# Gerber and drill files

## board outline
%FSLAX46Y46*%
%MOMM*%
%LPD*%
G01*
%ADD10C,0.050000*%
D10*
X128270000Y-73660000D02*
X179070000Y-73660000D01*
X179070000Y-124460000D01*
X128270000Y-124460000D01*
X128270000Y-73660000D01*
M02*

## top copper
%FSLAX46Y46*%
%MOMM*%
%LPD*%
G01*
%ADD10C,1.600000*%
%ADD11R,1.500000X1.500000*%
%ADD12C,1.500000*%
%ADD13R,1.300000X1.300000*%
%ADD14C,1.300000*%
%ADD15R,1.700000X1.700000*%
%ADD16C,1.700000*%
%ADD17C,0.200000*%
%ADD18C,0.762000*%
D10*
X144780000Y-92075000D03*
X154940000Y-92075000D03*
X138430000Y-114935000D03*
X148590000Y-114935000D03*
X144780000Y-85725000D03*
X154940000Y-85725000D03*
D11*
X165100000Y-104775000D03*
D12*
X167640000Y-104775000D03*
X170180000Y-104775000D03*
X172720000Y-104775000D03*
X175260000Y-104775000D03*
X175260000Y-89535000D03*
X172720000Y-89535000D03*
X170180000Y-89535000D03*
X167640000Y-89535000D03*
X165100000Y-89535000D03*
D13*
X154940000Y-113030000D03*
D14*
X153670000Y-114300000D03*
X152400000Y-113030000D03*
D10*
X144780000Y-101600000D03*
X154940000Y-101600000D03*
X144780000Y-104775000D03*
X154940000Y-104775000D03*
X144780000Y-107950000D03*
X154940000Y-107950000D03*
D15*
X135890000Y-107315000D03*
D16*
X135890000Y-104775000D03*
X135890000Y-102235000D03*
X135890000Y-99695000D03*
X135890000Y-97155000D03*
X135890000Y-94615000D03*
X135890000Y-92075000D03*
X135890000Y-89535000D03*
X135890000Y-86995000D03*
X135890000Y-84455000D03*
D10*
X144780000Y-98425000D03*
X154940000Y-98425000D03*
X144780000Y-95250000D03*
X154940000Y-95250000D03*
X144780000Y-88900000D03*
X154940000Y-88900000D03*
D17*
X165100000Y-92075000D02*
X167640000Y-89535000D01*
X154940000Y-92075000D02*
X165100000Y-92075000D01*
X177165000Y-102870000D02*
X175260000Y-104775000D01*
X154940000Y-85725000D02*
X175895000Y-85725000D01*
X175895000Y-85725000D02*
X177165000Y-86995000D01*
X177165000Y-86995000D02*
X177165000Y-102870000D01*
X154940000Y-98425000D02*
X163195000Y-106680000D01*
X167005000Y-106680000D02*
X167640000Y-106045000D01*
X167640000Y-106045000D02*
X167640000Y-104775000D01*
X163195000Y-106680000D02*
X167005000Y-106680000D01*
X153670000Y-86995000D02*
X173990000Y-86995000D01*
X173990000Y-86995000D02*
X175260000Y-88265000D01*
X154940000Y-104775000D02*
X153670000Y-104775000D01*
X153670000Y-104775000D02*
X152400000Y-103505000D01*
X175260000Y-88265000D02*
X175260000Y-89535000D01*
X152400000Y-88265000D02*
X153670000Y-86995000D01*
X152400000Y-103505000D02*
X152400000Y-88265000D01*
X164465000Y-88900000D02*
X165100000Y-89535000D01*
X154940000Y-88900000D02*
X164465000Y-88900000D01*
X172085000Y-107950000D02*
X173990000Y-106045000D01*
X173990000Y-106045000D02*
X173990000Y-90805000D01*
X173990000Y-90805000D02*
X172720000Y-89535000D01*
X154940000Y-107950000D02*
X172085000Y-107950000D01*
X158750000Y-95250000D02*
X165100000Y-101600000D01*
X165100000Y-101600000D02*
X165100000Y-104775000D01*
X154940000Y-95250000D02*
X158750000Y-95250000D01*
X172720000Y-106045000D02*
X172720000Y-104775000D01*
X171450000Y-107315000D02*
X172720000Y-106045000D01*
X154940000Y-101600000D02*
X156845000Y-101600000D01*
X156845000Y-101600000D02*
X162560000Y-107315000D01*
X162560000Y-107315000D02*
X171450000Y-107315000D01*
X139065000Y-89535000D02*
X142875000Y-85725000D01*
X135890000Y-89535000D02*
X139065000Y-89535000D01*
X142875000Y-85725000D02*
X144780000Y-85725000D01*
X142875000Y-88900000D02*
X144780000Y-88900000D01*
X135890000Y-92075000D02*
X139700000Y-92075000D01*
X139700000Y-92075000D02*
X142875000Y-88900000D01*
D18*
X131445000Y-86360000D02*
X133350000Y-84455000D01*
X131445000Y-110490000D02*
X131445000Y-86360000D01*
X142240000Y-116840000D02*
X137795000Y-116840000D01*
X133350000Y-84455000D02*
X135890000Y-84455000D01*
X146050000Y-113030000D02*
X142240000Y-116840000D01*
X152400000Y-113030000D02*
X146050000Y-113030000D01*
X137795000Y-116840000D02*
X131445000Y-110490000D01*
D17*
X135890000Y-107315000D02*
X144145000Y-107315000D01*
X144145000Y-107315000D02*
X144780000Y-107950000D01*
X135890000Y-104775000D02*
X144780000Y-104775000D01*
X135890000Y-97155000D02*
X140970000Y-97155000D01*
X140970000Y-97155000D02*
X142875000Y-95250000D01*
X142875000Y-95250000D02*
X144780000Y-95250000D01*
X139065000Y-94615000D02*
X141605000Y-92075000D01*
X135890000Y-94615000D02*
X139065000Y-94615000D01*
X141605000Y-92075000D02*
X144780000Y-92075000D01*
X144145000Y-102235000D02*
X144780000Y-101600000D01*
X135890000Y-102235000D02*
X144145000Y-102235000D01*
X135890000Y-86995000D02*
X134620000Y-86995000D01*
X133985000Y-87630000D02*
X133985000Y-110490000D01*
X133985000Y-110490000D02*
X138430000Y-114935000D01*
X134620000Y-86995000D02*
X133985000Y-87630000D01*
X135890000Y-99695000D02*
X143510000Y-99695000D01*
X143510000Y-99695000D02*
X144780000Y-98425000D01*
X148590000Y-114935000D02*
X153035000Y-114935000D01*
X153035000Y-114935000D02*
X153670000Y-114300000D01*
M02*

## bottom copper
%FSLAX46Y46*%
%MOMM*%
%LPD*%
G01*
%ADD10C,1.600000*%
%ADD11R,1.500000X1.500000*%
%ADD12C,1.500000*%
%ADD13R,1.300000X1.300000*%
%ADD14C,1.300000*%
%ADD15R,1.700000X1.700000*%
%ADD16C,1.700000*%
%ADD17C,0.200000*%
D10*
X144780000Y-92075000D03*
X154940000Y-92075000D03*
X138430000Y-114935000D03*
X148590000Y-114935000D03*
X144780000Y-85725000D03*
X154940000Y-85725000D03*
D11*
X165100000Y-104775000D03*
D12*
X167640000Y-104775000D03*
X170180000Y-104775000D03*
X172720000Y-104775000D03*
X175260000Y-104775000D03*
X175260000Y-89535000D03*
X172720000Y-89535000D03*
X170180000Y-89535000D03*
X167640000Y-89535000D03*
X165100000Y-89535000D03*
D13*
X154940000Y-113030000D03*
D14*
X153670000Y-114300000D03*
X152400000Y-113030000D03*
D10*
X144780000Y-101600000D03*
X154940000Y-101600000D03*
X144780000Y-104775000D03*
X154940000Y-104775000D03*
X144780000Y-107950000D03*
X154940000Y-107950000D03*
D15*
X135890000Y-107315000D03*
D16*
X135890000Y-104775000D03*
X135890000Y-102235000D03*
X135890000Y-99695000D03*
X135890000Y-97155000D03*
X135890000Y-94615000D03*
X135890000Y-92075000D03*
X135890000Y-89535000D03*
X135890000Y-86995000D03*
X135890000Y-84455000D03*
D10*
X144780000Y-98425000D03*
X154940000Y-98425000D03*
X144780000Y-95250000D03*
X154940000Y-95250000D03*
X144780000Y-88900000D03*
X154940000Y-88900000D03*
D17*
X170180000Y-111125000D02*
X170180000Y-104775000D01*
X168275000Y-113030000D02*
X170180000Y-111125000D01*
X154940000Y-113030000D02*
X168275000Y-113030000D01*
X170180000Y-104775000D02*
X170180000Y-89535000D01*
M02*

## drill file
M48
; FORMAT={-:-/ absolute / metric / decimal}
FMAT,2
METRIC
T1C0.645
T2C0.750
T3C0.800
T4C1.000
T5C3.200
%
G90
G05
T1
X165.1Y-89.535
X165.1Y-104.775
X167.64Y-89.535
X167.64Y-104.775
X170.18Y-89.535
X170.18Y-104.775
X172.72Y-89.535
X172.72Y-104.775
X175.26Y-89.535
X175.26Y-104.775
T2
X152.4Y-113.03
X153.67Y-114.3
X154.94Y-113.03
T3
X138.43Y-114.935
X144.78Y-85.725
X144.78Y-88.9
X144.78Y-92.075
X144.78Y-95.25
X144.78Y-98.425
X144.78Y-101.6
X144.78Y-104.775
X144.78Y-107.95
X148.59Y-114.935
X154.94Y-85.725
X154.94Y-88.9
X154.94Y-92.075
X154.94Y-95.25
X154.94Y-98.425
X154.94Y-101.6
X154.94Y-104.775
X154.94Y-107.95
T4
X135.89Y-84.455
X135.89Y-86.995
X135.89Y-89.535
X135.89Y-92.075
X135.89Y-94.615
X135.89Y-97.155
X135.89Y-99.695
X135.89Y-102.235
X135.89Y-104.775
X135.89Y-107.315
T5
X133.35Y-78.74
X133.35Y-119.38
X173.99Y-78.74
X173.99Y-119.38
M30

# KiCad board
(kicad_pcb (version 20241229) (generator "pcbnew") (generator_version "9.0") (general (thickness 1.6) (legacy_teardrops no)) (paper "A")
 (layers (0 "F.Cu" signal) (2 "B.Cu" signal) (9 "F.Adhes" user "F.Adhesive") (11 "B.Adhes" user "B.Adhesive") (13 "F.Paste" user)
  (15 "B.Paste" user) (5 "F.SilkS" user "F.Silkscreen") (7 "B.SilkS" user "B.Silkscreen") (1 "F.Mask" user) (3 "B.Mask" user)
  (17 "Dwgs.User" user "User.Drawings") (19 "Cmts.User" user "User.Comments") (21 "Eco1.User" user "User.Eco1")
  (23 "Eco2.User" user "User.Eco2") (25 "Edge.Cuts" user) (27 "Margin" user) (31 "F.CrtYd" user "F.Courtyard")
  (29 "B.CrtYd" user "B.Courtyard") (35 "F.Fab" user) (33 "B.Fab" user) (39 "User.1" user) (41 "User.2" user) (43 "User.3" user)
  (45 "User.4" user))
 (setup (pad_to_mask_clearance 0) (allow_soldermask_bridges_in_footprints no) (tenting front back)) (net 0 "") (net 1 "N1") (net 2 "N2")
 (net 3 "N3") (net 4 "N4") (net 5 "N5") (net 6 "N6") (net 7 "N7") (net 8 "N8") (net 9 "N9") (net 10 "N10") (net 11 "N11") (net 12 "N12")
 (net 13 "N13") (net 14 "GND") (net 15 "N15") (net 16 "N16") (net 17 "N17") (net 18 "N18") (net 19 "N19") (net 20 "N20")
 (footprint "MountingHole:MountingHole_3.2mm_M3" (layer "F.Cu") (at 133.35 78.74)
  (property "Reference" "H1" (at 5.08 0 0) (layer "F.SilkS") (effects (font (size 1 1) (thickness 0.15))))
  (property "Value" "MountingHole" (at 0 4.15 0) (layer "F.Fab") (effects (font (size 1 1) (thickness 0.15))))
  (pad "" np_thru_hole circle (at 0 0) (size 3.2 3.2) (drill 3.2) (layers "*.Cu" "*.Mask")))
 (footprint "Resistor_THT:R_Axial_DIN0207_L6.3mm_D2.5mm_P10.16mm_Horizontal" (layer "F.Cu") (at 144.78 92.075)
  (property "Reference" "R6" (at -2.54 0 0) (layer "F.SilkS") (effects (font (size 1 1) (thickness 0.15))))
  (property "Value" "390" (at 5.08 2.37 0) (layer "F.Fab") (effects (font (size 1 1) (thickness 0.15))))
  (pad "1" thru_hole circle (at 0 0) (size 1.6 1.6) (drill 0.8) (layers "*.Cu" "*.Mask") (remove_unused_layers no) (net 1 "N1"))
  (pad "2" thru_hole circle (at 10.16 0) (size 1.6 1.6) (drill 0.8) (layers "*.Cu" "*.Mask") (remove_unused_layers no) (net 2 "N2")))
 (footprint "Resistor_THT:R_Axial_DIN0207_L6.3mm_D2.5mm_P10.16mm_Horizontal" (layer "F.Cu") (at 138.43 114.935)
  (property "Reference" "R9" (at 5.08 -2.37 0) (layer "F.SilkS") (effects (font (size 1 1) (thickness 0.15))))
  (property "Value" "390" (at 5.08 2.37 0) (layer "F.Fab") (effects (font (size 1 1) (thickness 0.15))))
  (pad "1" thru_hole circle (at 0 0) (size 1.6 1.6) (drill 0.8) (layers "*.Cu" "*.Mask") (remove_unused_layers no) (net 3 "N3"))
  (pad "2" thru_hole circle (at 10.16 0) (size 1.6 1.6) (drill 0.8) (layers "*.Cu" "*.Mask") (remove_unused_layers no) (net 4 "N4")))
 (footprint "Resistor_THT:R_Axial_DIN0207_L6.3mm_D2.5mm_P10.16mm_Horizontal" (layer "F.Cu") (at 144.78 85.725)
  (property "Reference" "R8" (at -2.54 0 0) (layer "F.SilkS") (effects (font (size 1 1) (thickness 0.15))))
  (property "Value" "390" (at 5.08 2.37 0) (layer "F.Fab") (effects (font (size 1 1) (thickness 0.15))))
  (pad "1" thru_hole circle (at 0 0) (size 1.6 1.6) (drill 0.8) (layers "*.Cu" "*.Mask") (remove_unused_layers no) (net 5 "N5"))
  (pad "2" thru_hole circle (at 10.16 0) (size 1.6 1.6) (drill 0.8) (layers "*.Cu" "*.Mask") (remove_unused_layers no) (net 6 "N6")))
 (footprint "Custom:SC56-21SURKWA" (layer "F.Cu") (at 170.18 97.155)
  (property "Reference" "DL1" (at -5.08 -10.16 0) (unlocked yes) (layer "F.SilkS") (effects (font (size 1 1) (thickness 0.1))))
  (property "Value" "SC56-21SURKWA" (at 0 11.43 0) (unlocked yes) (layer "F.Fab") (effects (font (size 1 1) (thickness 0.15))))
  (pad "1" thru_hole rect (at -5.08 7.62 90) (size 1.5 1.5) (drill 0.64516) (layers "*.Cu" "*.Mask") (remove_unused_layers no) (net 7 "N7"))
  (pad "2" thru_hole circle (at -2.54 7.62 90) (size 1.5 1.5) (drill 0.64516) (layers "*.Cu" "*.Mask") (remove_unused_layers no)
   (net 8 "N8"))
  (pad "3" thru_hole circle (at 0 7.62 90) (size 1.5 1.5) (drill 0.64516) (layers "*.Cu" "*.Mask") (remove_unused_layers no) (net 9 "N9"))
  (pad "4" thru_hole circle (at 2.54 7.62 90) (size 1.5 1.5) (drill 0.64516) (layers "*.Cu" "*.Mask") (remove_unused_layers no)
   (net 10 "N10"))
  (pad "5" thru_hole circle (at 5.08 7.62 90) (size 1.5 1.5) (drill 0.64516) (layers "*.Cu" "*.Mask") (remove_unused_layers no) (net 6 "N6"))
  (pad "6" thru_hole circle (at 5.08 -7.62 90) (size 1.5 1.5) (drill 0.64516) (layers "*.Cu" "*.Mask") (remove_unused_layers no)
   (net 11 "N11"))
  (pad "7" thru_hole circle (at 2.54 -7.62 90) (size 1.5 1.5) (drill 0.64516) (layers "*.Cu" "*.Mask") (remove_unused_layers no)
   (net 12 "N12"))
  (pad "8" thru_hole circle (at 0 -7.62 90) (size 1.5 1.5) (drill 0.64516) (layers "*.Cu" "*.Mask") (remove_unused_layers no) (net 9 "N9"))
  (pad "9" thru_hole circle (at -2.54 -7.62 90) (size 1.5 1.5) (drill 0.64516) (layers "*.Cu" "*.Mask") (remove_unused_layers no)
   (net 2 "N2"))
  (pad "10" thru_hole circle (at -5.08 -7.62 90) (size 1.5 1.5) (drill 0.64516) (layers "*.Cu" "*.Mask") (remove_unused_layers no)
   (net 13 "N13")))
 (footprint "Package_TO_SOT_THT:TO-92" (layer "F.Cu") (at 154.94 113.03 180)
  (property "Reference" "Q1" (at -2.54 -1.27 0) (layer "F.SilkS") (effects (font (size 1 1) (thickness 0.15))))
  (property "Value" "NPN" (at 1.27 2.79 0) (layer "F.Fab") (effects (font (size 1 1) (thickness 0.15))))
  (pad "1" thru_hole rect (at 0 0 180) (size 1.3 1.3) (drill 0.75) (layers "*.Cu" "*.Mask") (remove_unused_layers no) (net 9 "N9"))
  (pad "2" thru_hole circle (at 1.27 -1.27 180) (size 1.3 1.3) (drill 0.75) (layers "*.Cu" "*.Mask") (remove_unused_layers no) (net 4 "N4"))
  (pad "3" thru_hole circle (at 2.54 0 180) (size 1.3 1.3) (drill 0.75) (layers "*.Cu" "*.Mask") (remove_unused_layers no) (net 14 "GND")))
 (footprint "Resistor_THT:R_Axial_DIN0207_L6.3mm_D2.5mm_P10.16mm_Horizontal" (layer "F.Cu") (at 144.78 101.6)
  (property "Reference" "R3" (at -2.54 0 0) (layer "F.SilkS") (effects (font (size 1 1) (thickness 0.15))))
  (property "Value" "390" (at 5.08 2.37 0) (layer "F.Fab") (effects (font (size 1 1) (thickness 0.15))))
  (pad "1" thru_hole circle (at 0 0) (size 1.6 1.6) (drill 0.8) (layers "*.Cu" "*.Mask") (remove_unused_layers no) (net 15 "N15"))
  (pad "2" thru_hole circle (at 10.16 0) (size 1.6 1.6) (drill 0.8) (layers "*.Cu" "*.Mask") (remove_unused_layers no) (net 10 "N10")))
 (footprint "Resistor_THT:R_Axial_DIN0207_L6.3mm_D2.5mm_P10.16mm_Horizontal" (layer "F.Cu") (at 144.78 104.775)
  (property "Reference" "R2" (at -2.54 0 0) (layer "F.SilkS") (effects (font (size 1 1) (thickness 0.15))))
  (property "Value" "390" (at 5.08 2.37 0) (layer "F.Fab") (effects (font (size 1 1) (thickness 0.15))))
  (pad "1" thru_hole circle (at 0 0) (size 1.6 1.6) (drill 0.8) (layers "*.Cu" "*.Mask") (remove_unused_layers no) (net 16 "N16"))
  (pad "2" thru_hole circle (at 10.16 0) (size 1.6 1.6) (drill 0.8) (layers "*.Cu" "*.Mask") (remove_unused_layers no) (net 11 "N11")))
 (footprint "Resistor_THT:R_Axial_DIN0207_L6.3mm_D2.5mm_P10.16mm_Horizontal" (layer "F.Cu") (at 144.78 107.95)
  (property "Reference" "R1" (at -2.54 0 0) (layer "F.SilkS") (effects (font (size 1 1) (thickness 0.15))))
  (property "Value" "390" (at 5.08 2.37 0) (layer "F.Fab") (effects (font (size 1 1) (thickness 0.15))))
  (pad "1" thru_hole circle (at 0 0) (size 1.6 1.6) (drill 0.8) (layers "*.Cu" "*.Mask") (remove_unused_layers no) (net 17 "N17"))
  (pad "2" thru_hole circle (at 10.16 0) (size 1.6 1.6) (drill 0.8) (layers "*.Cu" "*.Mask") (remove_unused_layers no) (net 12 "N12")))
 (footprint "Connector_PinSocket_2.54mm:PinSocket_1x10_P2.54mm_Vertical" (layer "F.Cu") (at 135.89 107.315 180)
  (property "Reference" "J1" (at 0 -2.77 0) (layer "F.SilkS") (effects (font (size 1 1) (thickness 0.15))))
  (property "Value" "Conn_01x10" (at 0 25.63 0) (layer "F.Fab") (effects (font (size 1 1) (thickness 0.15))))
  (pad "1" thru_hole rect (at 0 0 180) (size 1.7 1.7) (drill 1) (layers "*.Cu" "*.Mask") (remove_unused_layers no) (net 17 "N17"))
  (pad "2" thru_hole circle (at 0 2.54 180) (size 1.7 1.7) (drill 1) (layers "*.Cu" "*.Mask") (remove_unused_layers no) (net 16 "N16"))
  (pad "3" thru_hole circle (at 0 5.08 180) (size 1.7 1.7) (drill 1) (layers "*.Cu" "*.Mask") (remove_unused_layers no) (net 15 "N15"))
  (pad "4" thru_hole circle (at 0 7.62 180) (size 1.7 1.7) (drill 1) (layers "*.Cu" "*.Mask") (remove_unused_layers no) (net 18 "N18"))
  (pad "5" thru_hole circle (at 0 10.16 180) (size 1.7 1.7) (drill 1) (layers "*.Cu" "*.Mask") (remove_unused_layers no) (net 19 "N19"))
  (pad "6" thru_hole circle (at 0 12.7 180) (size 1.7 1.7) (drill 1) (layers "*.Cu" "*.Mask") (remove_unused_layers no) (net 1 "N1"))
  (pad "7" thru_hole circle (at 0 15.24 180) (size 1.7 1.7) (drill 1) (layers "*.Cu" "*.Mask") (remove_unused_layers no) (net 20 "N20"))
  (pad "8" thru_hole circle (at 0 17.78 180) (size 1.7 1.7) (drill 1) (layers "*.Cu" "*.Mask") (remove_unused_layers no) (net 5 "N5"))
  (pad "9" thru_hole circle (at 0 20.32 180) (size 1.7 1.7) (drill 1) (layers "*.Cu" "*.Mask") (remove_unused_layers no) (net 3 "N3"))
  (pad "10" thru_hole circle (at 0 22.86 180) (size 1.7 1.7) (drill 1) (layers "*.Cu" "*.Mask") (remove_unused_layers no) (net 14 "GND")))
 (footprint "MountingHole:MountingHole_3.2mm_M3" (layer "F.Cu") (at 173.99 78.74)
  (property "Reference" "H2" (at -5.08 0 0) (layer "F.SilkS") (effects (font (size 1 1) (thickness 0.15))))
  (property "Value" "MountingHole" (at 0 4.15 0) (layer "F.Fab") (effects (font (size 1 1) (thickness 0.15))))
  (pad "" np_thru_hole circle (at 0 0) (size 3.2 3.2) (drill 3.2) (layers "*.Cu" "*.Mask")))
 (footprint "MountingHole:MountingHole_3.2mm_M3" (layer "F.Cu") (at 173.99 119.38)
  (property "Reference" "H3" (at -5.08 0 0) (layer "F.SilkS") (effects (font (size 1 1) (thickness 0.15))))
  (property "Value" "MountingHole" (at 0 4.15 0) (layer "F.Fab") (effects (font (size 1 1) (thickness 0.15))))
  (pad "" np_thru_hole circle (at 0 0) (size 3.2 3.2) (drill 3.2) (layers "*.Cu" "*.Mask")))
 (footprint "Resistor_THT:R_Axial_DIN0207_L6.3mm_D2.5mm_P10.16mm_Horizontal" (layer "F.Cu") (at 144.78 98.425)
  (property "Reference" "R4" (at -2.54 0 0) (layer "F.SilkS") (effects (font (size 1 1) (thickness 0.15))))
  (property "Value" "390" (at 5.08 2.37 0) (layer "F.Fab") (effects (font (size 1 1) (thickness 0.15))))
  (pad "1" thru_hole circle (at 0 0) (size 1.6 1.6) (drill 0.8) (layers "*.Cu" "*.Mask") (remove_unused_layers no) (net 18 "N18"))
  (pad "2" thru_hole circle (at 10.16 0) (size 1.6 1.6) (drill 0.8) (layers "*.Cu" "*.Mask") (remove_unused_layers no) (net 8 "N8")))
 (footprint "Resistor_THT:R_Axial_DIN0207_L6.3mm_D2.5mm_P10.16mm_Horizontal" (layer "F.Cu") (at 144.78 95.25)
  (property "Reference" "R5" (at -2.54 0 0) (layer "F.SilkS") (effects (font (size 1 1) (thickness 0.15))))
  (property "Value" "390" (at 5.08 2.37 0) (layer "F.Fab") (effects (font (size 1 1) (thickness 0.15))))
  (pad "1" thru_hole circle (at 0 0) (size 1.6 1.6) (drill 0.8) (layers "*.Cu" "*.Mask") (remove_unused_layers no) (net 19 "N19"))
  (pad "2" thru_hole circle (at 10.16 0) (size 1.6 1.6) (drill 0.8) (layers "*.Cu" "*.Mask") (remove_unused_layers no) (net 7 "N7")))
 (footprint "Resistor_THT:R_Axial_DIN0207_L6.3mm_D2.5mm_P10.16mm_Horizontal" (layer "F.Cu") (at 144.78 88.9)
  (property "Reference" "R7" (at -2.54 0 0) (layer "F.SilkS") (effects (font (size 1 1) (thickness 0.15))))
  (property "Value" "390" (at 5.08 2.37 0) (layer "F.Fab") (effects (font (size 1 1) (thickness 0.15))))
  (pad "1" thru_hole circle (at 0 0) (size 1.6 1.6) (drill 0.8) (layers "*.Cu" "*.Mask") (remove_unused_layers no) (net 20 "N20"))
  (pad "2" thru_hole circle (at 10.16 0) (size 1.6 1.6) (drill 0.8) (layers "*.Cu" "*.Mask") (remove_unused_layers no) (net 13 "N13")))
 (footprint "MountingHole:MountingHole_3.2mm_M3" (layer "F.Cu") (at 133.35 119.38)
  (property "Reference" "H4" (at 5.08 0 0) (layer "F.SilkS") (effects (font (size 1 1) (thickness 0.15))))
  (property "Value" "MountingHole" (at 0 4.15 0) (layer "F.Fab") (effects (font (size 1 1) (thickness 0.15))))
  (pad "" np_thru_hole circle (at 0 0) (size 3.2 3.2) (drill 3.2) (layers "*.Cu" "*.Mask")))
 (gr_rect (start 128.27 73.66) (end 179.07 124.46) (stroke (width 0.05) (type default)) (fill no) (layer "Edge.Cuts"))
 (segment (start 165.1 92.075) (end 167.64 89.535) (width 0.2) (layer "F.Cu") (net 2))
 (segment (start 154.94 92.075) (end 165.1 92.075) (width 0.2) (layer "F.Cu") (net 2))
 (segment (start 177.165 102.87) (end 175.26 104.775) (width 0.2) (layer "F.Cu") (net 6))
 (segment (start 154.94 85.725) (end 175.895 85.725) (width 0.2) (layer "F.Cu") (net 6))
 (segment (start 175.895 85.725) (end 177.165 86.995) (width 0.2) (layer "F.Cu") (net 6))
 (segment (start 177.165 86.995) (end 177.165 102.87) (width 0.2) (layer "F.Cu") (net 6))
 (segment (start 170.18 111.125) (end 170.18 104.775) (width 0.2) (layer "B.Cu") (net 9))
 (segment (start 168.275 113.03) (end 170.18 111.125) (width 0.2) (layer "B.Cu") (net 9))
 (segment (start 154.94 113.03) (end 168.275 113.03) (width 0.2) (layer "B.Cu") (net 9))
 (segment (start 170.18 104.775) (end 170.18 89.535) (width 0.2) (layer "B.Cu") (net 9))
 (segment (start 154.94 98.425) (end 163.195 106.68) (width 0.2) (layer "F.Cu") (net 8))
 (segment (start 167.005 106.68) (end 167.64 106.045) (width 0.2) (layer "F.Cu") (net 8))
 (segment (start 167.64 106.045) (end 167.64 104.775) (width 0.2) (layer "F.Cu") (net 8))
 (segment (start 163.195 106.68) (end 167.005 106.68) (width 0.2) (layer "F.Cu") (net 8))
 (segment (start 153.67 86.995) (end 173.99 86.995) (width 0.2) (layer "F.Cu") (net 11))
 (segment (start 173.99 86.995) (end 175.26 88.265) (width 0.2) (layer "F.Cu") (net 11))
 (segment (start 154.94 104.775) (end 153.67 104.775) (width 0.2) (layer "F.Cu") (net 11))
 (segment (start 153.67 104.775) (end 152.4 103.505) (width 0.2) (layer "F.Cu") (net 11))
 (segment (start 175.26 88.265) (end 175.26 89.535) (width 0.2) (layer "F.Cu") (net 11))
 (segment (start 152.4 88.265) (end 153.67 86.995) (width 0.2) (layer "F.Cu") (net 11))
 (segment (start 152.4 103.505) (end 152.4 88.265) (width 0.2) (layer "F.Cu") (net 11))
 (segment (start 164.465 88.9) (end 165.1 89.535) (width 0.2) (layer "F.Cu") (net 13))
 (segment (start 154.94 88.9) (end 164.465 88.9) (width 0.2) (layer "F.Cu") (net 13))
 (segment (start 172.085 107.95) (end 173.99 106.045) (width 0.2) (layer "F.Cu") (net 12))
 (segment (start 173.99 106.045) (end 173.99 90.805) (width 0.2) (layer "F.Cu") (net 12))
 (segment (start 173.99 90.805) (end 172.72 89.535) (width 0.2) (layer "F.Cu") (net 12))
 (segment (start 154.94 107.95) (end 172.085 107.95) (width 0.2) (layer "F.Cu") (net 12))
 (segment (start 158.75 95.25) (end 165.1 101.6) (width 0.2) (layer "F.Cu") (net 7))
 (segment (start 165.1 101.6) (end 165.1 104.775) (width 0.2) (layer "F.Cu") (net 7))
 (segment (start 154.94 95.25) (end 158.75 95.25) (width 0.2) (layer "F.Cu") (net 7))
 (segment (start 172.72 106.045) (end 172.72 104.775) (width 0.2) (layer "F.Cu") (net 10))
 (segment (start 171.45 107.315) (end 172.72 106.045) (width 0.2) (layer "F.Cu") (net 10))
 (segment (start 154.94 101.6) (end 156.845 101.6) (width 0.2) (layer "F.Cu") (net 10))
 (segment (start 156.845 101.6) (end 162.56 107.315) (width 0.2) (layer "F.Cu") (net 10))
 (segment (start 162.56 107.315) (end 171.45 107.315) (width 0.2) (layer "F.Cu") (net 10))
 (segment (start 139.065 89.535) (end 142.875 85.725) (width 0.2) (layer "F.Cu") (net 5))
 (segment (start 135.89 89.535) (end 139.065 89.535) (width 0.2) (layer "F.Cu") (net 5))
 (segment (start 142.875 85.725) (end 144.78 85.725) (width 0.2) (layer "F.Cu") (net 5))
 (segment (start 142.875 88.9) (end 144.78 88.9) (width 0.2) (layer "F.Cu") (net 20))
 (segment (start 135.89 92.075) (end 139.7 92.075) (width 0.2) (layer "F.Cu") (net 20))
 (segment (start 139.7 92.075) (end 142.875 88.9) (width 0.2) (layer "F.Cu") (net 20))
 (segment (start 131.445 86.36) (end 133.35 84.455) (width 0.762) (layer "F.Cu") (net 14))
 (segment (start 131.445 110.49) (end 131.445 86.36) (width 0.762) (layer "F.Cu") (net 14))
 (segment (start 142.24 116.84) (end 137.795 116.84) (width 0.762) (layer "F.Cu") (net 14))
 (segment (start 133.35 84.455) (end 135.89 84.455) (width 0.762) (layer "F.Cu") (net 14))
 (segment (start 146.05 113.03) (end 142.24 116.84) (width 0.762) (layer "F.Cu") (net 14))
 (segment (start 152.4 113.03) (end 146.05 113.03) (width 0.762) (layer "F.Cu") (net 14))
 (segment (start 137.795 116.84) (end 131.445 110.49) (width 0.762) (layer "F.Cu") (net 14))
 (segment (start 135.89 107.315) (end 144.145 107.315) (width 0.2) (layer "F.Cu") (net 17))
 (segment (start 144.145 107.315) (end 144.78 107.95) (width 0.2) (layer "F.Cu") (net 17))
 (segment (start 135.89 104.775) (end 144.78 104.775) (width 0.2) (layer "F.Cu") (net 16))
 (segment (start 135.89 97.155) (end 140.97 97.155) (width 0.2) (layer "F.Cu") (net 19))
 (segment (start 140.97 97.155) (end 142.875 95.25) (width 0.2) (layer "F.Cu") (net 19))
 (segment (start 142.875 95.25) (end 144.78 95.25) (width 0.2) (layer "F.Cu") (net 19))
 (segment (start 139.065 94.615) (end 141.605 92.075) (width 0.2) (layer "F.Cu") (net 1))
 (segment (start 135.89 94.615) (end 139.065 94.615) (width 0.2) (layer "F.Cu") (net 1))
 (segment (start 141.605 92.075) (end 144.78 92.075) (width 0.2) (layer "F.Cu") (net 1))
 (segment (start 144.145 102.235) (end 144.78 101.6) (width 0.2) (layer "F.Cu") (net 15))
 (segment (start 135.89 102.235) (end 144.145 102.235) (width 0.2) (layer "F.Cu") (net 15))
 (segment (start 135.89 86.995) (end 134.62 86.995) (width 0.2) (layer "F.Cu") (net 3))
 (segment (start 133.985 87.63) (end 133.985 110.49) (width 0.2) (layer "F.Cu") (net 3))
 (segment (start 133.985 110.49) (end 138.43 114.935) (width 0.2) (layer "F.Cu") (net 3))
 (segment (start 134.62 86.995) (end 133.985 87.63) (width 0.2) (layer "F.Cu") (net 3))
 (segment (start 135.89 99.695) (end 143.51 99.695) (width 0.2) (layer "F.Cu") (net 18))
 (segment (start 143.51 99.695) (end 144.78 98.425) (width 0.2) (layer "F.Cu") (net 18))
 (segment (start 148.59 114.935) (end 153.035 114.935) (width 0.2) (layer "F.Cu") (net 4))
 (segment (start 153.035 114.935) (end 153.67 114.3) (width 0.2) (layer "F.Cu") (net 4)))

